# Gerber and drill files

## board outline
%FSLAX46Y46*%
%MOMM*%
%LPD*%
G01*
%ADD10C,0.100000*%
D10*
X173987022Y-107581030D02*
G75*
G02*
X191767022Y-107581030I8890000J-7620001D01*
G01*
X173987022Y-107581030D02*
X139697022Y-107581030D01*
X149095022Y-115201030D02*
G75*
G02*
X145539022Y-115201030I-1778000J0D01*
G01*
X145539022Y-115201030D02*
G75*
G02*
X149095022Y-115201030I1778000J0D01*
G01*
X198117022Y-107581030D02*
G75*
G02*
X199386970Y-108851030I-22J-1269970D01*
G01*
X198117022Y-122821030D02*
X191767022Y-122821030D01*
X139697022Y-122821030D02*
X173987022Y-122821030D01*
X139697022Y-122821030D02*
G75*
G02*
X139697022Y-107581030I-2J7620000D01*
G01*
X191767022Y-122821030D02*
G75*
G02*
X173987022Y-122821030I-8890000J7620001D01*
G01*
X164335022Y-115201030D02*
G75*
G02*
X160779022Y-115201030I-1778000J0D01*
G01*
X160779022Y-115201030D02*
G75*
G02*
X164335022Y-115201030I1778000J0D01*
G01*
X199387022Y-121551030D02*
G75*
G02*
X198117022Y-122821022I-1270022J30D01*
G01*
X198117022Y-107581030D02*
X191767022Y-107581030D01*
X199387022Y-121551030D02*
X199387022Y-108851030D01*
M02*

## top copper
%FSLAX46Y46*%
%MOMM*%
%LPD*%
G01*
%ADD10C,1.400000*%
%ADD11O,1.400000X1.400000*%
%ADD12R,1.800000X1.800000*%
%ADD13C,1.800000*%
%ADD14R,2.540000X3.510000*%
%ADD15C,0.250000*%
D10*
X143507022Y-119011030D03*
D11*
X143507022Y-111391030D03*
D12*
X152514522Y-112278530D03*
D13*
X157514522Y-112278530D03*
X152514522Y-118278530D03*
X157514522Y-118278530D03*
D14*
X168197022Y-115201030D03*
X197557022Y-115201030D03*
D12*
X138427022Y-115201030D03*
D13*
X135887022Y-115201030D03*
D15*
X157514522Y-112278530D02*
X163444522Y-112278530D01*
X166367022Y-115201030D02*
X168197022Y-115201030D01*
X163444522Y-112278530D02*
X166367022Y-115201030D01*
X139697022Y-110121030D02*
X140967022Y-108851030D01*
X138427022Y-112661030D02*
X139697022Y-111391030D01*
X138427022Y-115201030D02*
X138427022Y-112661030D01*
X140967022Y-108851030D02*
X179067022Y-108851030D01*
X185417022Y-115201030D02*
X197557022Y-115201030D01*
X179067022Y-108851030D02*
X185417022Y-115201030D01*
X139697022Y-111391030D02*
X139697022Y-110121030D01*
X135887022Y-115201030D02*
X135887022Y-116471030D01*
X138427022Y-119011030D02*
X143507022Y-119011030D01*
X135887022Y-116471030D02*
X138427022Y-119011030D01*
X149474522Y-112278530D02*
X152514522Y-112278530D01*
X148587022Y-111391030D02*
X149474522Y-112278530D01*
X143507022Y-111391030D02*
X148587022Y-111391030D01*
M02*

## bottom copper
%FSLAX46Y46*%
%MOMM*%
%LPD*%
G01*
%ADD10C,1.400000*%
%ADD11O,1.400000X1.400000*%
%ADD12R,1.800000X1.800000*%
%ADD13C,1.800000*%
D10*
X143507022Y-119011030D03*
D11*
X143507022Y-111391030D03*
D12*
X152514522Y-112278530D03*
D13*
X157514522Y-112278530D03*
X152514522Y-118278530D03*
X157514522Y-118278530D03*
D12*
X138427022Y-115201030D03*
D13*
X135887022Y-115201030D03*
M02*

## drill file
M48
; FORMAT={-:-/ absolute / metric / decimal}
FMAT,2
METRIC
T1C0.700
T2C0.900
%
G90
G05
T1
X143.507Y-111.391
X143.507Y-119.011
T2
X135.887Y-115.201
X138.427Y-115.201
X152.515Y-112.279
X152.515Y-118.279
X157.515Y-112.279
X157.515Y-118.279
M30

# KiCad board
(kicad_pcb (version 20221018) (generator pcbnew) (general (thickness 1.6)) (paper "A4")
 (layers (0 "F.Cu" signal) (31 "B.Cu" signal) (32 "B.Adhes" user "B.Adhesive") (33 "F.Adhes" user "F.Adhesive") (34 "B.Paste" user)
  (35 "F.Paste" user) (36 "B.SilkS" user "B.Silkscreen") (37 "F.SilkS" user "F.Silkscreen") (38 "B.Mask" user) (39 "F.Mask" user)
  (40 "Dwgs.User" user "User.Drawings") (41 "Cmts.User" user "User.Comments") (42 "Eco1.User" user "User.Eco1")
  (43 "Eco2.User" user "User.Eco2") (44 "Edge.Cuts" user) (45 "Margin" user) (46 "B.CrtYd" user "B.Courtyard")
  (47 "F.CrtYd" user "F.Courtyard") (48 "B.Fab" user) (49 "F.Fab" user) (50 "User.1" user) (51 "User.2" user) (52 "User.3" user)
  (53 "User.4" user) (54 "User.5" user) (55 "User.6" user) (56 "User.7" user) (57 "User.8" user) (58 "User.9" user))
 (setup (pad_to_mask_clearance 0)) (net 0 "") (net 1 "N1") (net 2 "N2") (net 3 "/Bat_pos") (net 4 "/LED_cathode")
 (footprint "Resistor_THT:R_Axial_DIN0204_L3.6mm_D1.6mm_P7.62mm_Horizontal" (layer "F.Cu") (at 143.507022 119.01103 90)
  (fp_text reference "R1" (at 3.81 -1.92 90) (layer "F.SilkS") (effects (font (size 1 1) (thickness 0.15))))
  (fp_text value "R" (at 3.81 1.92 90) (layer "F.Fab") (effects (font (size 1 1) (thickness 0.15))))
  (pad "1" thru_hole circle (at 0 0 90) (size 1.4 1.4) (drill 0.7) (layers "*.Cu" "*.Mask") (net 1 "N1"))
  (pad "2" thru_hole oval (at 7.62 0 90) (size 1.4 1.4) (drill 0.7) (layers "*.Cu" "*.Mask") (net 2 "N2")))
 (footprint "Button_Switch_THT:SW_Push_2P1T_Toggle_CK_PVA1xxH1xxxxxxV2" (layer "F.Cu") (at 152.514522 112.27853)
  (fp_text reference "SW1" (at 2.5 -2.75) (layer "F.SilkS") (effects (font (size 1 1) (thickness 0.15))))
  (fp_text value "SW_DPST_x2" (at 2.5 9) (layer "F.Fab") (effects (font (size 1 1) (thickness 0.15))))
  (pad "1" thru_hole rect (at 0 0) (size 1.8 1.8) (drill 0.9) (layers "*.Cu" "*.Mask") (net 2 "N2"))
  (pad "2" thru_hole circle (at 5 0) (size 1.8 1.8) (drill 0.9) (layers "*.Cu" "*.Mask") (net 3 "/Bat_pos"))
  (pad "3" thru_hole circle (at 0 6) (size 1.8 1.8) (drill 0.9) (layers "*.Cu" "*.Mask"))
  (pad "4" thru_hole circle (at 5 6) (size 1.8 1.8) (drill 0.9) (layers "*.Cu" "*.Mask")))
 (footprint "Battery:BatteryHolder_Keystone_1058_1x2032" (layer "F.Cu") (at 182.877022 115.20103)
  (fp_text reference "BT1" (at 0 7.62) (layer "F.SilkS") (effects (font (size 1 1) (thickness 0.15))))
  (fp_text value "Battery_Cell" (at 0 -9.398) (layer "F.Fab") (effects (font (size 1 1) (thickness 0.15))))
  (pad "1" smd rect (at -14.68 0) (size 2.54 3.51) (layers "F.Cu" "F.Paste" "F.Mask") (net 3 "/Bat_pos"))
  (pad "2" smd rect (at 14.68 0) (size 2.54 3.51) (layers "F.Cu" "F.Paste" "F.Mask") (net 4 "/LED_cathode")))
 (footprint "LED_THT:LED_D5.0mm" (layer "F.Cu") (at 138.427022 115.20103 180)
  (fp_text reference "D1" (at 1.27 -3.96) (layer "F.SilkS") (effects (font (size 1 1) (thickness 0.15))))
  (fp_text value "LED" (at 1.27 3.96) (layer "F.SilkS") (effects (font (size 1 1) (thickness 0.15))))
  (pad "1" thru_hole rect (at 0 0 180) (size 1.8 1.8) (drill 0.9) (layers "*.Cu" "*.Mask") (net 4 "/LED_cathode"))
  (pad "2" thru_hole circle (at 2.54 0 180) (size 1.8 1.8) (drill 0.9) (layers "*.Cu" "*.Mask") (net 1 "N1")))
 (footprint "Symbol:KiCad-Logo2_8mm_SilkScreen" (layer "B.Cu") (at 182.877022 113.93103 180)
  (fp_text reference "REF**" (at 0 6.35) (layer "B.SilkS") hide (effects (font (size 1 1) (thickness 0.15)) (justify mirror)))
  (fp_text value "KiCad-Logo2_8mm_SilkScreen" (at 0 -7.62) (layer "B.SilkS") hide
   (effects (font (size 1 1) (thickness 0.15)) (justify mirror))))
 (gr_arc (start 173.987022 107.58103) (mid 182.877022 103.492209) (end 191.767022 107.58103) (stroke (width 0.1) (type solid))
  (layer "Edge.Cuts"))
 (gr_line (start 173.987022 107.58103) (end 139.697022 107.58103) (stroke (width 0.1) (type solid)) (layer "Edge.Cuts"))
 (gr_circle (center 147.317022 115.20103) (end 149.095022 115.20103) (stroke (width 0.1) (type solid)) (fill none) (layer "Edge.Cuts"))
 (gr_arc (start 198.117022 107.58103) (mid 199.015048 107.953004) (end 199.387022 108.85103) (stroke (width 0.1) (type solid))
  (layer "Edge.Cuts"))
 (gr_line (start 198.117022 122.82103) (end 191.767022 122.82103) (stroke (width 0.1) (type solid)) (layer "Edge.Cuts"))
 (gr_line (start 139.697022 122.82103) (end 173.987022 122.82103) (stroke (width 0.1) (type solid)) (layer "Edge.Cuts"))
 (gr_arc (start 139.697022 122.82103) (mid 132.077022 115.20103) (end 139.697022 107.58103) (stroke (width 0.1) (type solid))
  (layer "Edge.Cuts"))
 (gr_arc (start 191.767022 122.82103) (mid 182.877022 126.909851) (end 173.987022 122.82103) (stroke (width 0.1) (type solid))
  (layer "Edge.Cuts"))
 (gr_circle (center 162.557022 115.20103) (end 164.335022 115.20103) (stroke (width 0.1) (type solid)) (fill none) (layer "Edge.Cuts"))
 (gr_arc (start 199.387022 121.55103) (mid 199.015048 122.449056) (end 198.117022 122.82103) (stroke (width 0.1) (type solid))
  (layer "Edge.Cuts"))
 (gr_line (start 198.117022 107.58103) (end 191.767022 107.58103) (stroke (width 0.1) (type solid)) (layer "Edge.Cuts"))
 (gr_line (start 199.387022 121.55103) (end 199.387022 108.85103) (stroke (width 0.1) (type solid)) (layer "Edge.Cuts"))
 (segment (start 157.514522 112.27853) (end 163.444522 112.27853) (width 0.25) (layer "F.Cu") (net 3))
 (segment (start 166.367022 115.20103) (end 168.197022 115.20103) (width 0.25) (layer "F.Cu") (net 3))
 (segment (start 163.444522 112.27853) (end 166.367022 115.20103) (width 0.25) (layer "F.Cu") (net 3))
 (segment (start 139.697022 110.12103) (end 140.967022 108.85103) (width 0.25) (layer "F.Cu") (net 4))
 (segment (start 138.427022 112.66103) (end 139.697022 111.39103) (width 0.25) (layer "F.Cu") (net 4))
 (segment (start 138.427022 115.20103) (end 138.427022 112.66103) (width 0.25) (layer "F.Cu") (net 4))
 (segment (start 140.967022 108.85103) (end 179.067022 108.85103) (width 0.25) (layer "F.Cu") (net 4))
 (segment (start 185.417022 115.20103) (end 197.557022 115.20103) (width 0.25) (layer "F.Cu") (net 4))
 (segment (start 179.067022 108.85103) (end 185.417022 115.20103) (width 0.25) (layer "F.Cu") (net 4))
 (segment (start 139.697022 111.39103) (end 139.697022 110.12103) (width 0.25) (layer "F.Cu") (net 4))
 (segment (start 135.887022 115.20103) (end 135.887022 116.47103) (width 0.25) (layer "F.Cu") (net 1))
 (segment (start 138.427022 119.01103) (end 143.507022 119.01103) (width 0.25) (layer "F.Cu") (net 1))
 (segment (start 135.887022 116.47103) (end 138.427022 119.01103) (width 0.25) (layer "F.Cu") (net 1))
 (segment (start 149.474522 112.27853) (end 152.514522 112.27853) (width 0.25) (layer "F.Cu") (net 2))
 (segment (start 148.587022 111.39103) (end 149.474522 112.27853) (width 0.25) (layer "F.Cu") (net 2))
 (segment (start 143.507022 111.39103) (end 148.587022 111.39103) (width 0.25) (layer "F.Cu") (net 2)))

